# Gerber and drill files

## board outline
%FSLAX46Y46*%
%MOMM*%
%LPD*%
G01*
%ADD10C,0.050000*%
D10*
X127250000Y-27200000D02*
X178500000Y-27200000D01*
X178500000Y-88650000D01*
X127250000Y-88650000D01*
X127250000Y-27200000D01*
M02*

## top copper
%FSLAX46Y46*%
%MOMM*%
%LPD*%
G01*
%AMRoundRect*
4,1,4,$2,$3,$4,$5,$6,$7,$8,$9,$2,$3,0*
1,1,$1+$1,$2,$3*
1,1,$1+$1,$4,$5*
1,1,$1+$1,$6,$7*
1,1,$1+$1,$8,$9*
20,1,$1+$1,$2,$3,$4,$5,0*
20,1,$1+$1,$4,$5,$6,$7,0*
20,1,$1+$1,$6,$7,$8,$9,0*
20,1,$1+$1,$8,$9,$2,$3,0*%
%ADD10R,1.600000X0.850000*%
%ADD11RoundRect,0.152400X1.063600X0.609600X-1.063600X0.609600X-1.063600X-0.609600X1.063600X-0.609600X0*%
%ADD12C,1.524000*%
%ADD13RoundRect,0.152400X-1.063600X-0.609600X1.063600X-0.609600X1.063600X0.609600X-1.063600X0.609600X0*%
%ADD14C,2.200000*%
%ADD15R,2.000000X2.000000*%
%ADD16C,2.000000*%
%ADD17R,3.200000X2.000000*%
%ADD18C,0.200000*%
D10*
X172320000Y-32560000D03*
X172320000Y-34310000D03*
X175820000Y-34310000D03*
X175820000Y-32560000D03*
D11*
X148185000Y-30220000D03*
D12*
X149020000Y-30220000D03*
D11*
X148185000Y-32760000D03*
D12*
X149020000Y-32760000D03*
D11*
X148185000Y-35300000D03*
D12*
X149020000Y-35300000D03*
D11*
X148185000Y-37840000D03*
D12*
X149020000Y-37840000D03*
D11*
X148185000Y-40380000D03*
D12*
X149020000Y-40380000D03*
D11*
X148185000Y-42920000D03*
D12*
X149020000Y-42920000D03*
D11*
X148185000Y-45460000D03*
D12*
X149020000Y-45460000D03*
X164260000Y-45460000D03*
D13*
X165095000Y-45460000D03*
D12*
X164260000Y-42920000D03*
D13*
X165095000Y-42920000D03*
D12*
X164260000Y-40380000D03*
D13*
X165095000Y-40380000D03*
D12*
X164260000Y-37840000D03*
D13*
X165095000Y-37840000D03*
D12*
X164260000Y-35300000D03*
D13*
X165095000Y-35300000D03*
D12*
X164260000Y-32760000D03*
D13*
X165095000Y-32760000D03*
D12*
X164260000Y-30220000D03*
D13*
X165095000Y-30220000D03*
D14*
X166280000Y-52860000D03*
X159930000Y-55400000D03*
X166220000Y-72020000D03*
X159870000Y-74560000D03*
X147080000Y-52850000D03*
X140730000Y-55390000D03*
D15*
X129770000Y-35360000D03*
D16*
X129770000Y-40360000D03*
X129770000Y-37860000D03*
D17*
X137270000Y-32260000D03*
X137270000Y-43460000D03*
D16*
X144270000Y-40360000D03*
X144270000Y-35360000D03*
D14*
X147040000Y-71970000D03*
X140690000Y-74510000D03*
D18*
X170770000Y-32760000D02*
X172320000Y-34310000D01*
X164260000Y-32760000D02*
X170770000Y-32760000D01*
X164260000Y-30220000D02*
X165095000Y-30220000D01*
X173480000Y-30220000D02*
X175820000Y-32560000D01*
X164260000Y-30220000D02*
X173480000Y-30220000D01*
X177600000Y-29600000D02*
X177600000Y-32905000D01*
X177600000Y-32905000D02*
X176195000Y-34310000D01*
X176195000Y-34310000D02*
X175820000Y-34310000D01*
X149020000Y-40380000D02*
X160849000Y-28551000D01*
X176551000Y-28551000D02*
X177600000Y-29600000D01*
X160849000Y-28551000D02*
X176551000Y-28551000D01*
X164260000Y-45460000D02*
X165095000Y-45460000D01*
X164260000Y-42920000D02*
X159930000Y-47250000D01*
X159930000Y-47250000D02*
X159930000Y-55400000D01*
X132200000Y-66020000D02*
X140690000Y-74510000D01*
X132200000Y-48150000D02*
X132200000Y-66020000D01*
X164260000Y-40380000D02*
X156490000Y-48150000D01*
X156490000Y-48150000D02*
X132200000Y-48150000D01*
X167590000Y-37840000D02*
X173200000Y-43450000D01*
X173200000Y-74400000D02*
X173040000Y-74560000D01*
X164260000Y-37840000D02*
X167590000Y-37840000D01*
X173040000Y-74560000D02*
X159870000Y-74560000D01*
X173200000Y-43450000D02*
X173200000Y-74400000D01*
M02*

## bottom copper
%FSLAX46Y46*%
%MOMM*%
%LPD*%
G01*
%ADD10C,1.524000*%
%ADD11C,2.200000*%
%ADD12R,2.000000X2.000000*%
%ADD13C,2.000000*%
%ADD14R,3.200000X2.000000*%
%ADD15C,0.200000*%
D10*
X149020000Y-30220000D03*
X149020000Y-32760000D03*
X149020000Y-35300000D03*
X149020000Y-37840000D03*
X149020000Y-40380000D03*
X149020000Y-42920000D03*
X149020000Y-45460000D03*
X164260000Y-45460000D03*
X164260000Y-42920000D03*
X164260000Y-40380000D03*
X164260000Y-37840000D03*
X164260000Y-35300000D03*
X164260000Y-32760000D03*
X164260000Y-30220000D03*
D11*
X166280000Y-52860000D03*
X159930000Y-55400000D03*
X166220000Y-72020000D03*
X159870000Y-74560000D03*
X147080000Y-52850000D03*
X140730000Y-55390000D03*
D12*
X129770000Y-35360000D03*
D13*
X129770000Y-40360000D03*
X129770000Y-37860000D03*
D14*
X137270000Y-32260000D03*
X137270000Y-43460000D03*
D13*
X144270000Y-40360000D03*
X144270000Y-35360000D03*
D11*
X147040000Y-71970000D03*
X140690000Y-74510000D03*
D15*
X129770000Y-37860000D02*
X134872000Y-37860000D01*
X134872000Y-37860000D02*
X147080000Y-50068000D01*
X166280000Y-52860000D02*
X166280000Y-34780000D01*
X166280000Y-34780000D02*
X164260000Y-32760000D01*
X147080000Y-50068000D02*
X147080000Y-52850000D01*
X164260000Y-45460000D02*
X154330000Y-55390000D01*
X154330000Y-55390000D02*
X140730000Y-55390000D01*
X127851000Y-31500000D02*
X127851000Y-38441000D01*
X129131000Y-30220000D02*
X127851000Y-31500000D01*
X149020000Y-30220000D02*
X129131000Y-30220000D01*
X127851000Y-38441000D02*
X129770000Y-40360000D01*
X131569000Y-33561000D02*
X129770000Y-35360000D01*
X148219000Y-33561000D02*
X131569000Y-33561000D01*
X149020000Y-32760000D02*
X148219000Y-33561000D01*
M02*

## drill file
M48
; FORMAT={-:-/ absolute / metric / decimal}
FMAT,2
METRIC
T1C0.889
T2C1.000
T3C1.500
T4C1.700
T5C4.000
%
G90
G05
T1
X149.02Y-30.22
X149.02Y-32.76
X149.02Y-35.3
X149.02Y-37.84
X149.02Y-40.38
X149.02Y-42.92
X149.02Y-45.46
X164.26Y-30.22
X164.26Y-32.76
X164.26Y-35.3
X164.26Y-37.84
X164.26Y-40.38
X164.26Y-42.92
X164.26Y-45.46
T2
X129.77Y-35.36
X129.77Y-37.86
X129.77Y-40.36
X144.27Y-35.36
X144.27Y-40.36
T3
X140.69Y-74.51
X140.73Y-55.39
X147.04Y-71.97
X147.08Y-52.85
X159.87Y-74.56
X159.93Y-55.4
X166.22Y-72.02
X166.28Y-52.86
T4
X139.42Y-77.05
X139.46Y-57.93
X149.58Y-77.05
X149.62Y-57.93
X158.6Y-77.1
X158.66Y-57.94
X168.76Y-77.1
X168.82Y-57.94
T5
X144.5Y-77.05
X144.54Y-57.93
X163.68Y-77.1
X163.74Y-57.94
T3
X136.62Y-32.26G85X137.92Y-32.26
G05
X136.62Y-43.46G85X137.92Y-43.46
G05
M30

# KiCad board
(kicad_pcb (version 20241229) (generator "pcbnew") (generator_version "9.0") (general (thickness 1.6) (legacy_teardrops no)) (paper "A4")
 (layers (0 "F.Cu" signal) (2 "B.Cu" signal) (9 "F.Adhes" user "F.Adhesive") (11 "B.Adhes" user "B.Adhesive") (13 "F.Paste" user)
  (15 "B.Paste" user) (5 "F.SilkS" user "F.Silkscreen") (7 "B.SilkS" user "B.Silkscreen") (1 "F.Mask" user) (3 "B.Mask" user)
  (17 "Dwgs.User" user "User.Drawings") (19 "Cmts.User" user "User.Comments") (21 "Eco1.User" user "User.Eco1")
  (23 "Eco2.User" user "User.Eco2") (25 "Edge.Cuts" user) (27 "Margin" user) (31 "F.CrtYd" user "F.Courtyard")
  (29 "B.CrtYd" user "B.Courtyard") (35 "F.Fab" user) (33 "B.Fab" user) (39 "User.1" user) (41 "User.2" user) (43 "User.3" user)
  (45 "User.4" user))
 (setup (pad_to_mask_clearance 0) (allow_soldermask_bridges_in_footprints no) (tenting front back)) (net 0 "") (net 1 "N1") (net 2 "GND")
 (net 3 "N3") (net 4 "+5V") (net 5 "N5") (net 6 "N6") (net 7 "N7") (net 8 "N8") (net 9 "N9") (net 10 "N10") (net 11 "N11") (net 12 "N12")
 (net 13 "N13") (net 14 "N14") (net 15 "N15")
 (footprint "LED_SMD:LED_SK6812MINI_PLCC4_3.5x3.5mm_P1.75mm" (layer "F.Cu") (at 174.07 33.435)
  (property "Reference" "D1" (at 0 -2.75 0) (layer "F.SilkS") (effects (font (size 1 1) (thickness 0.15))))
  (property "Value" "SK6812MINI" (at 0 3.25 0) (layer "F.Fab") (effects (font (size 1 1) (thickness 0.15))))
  (pad "1" smd rect (at -1.75 -0.875) (size 1.6 0.85) (layers "F.Cu" "F.Mask" "F.Paste") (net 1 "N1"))
  (pad "2" smd rect (at -1.75 0.875) (size 1.6 0.85) (layers "F.Cu" "F.Mask" "F.Paste") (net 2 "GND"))
  (pad "3" smd rect (at 1.75 0.875) (size 1.6 0.85) (layers "F.Cu" "F.Mask" "F.Paste") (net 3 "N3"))
  (pad "4" smd rect (at 1.75 -0.875) (size 1.6 0.85) (layers "F.Cu" "F.Mask" "F.Paste") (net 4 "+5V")))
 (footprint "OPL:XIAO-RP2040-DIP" (layer "F.Cu") (at 156.64 37.84)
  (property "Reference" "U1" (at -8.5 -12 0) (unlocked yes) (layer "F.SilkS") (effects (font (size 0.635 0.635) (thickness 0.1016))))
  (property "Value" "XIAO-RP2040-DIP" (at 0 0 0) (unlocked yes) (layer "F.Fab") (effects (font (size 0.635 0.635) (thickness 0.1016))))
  (pad "1" smd roundrect (at -8.455 -7.62 180) (size 2.432 1.524) (layers "F.Cu" "F.Mask") (roundrect_rratio 0.1) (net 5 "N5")
   (thermal_bridge_angle 45))
  (pad "1" thru_hole circle (at -7.62 -7.62 180) (size 1.524 1.524) (drill 0.889) (layers "*.Cu" "*.Mask") (remove_unused_layers no)
   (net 5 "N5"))
  (pad "2" smd roundrect (at -8.455 -5.08 180) (size 2.432 1.524) (layers "F.Cu" "F.Mask") (roundrect_rratio 0.1) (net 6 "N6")
   (thermal_bridge_angle 45))
  (pad "2" thru_hole circle (at -7.62 -5.08 180) (size 1.524 1.524) (drill 0.889) (layers "*.Cu" "*.Mask") (remove_unused_layers no)
   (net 6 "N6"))
  (pad "3" smd roundrect (at -8.455 -2.54 180) (size 2.432 1.524) (layers "F.Cu" "F.Mask") (roundrect_rratio 0.1) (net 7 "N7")
   (thermal_bridge_angle 45))
  (pad "3" thru_hole circle (at -7.62 -2.54 180) (size 1.524 1.524) (drill 0.889) (layers "*.Cu" "*.Mask") (remove_unused_layers no)
   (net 7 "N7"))
  (pad "4" smd roundrect (at -8.455 0 180) (size 2.432 1.524) (layers "F.Cu" "F.Mask") (roundrect_rratio 0.1) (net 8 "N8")
   (thermal_bridge_angle 45))
  (pad "4" thru_hole circle (at -7.62 0 180) (size 1.524 1.524) (drill 0.889) (layers "*.Cu" "*.Mask") (remove_unused_layers no)
   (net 8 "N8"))
  (pad "5" smd roundrect (at -8.455 2.54 180) (size 2.432 1.524) (layers "F.Cu" "F.Mask") (roundrect_rratio 0.1) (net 3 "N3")
   (thermal_bridge_angle 45))
  (pad "5" thru_hole circle (at -7.62 2.54 180) (size 1.524 1.524) (drill 0.889) (layers "*.Cu" "*.Mask") (remove_unused_layers no)
   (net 3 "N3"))
  (pad "6" smd roundrect (at -8.455 5.08 180) (size 2.432 1.524) (layers "F.Cu" "F.Mask") (roundrect_rratio 0.1) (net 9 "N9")
   (thermal_bridge_angle 45))
  (pad "6" thru_hole circle (at -7.62 5.08 180) (size 1.524 1.524) (drill 0.889) (layers "*.Cu" "*.Mask") (remove_unused_layers no)
   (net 9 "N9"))
  (pad "7" smd roundrect (at -8.455 7.62 180) (size 2.432 1.524) (layers "F.Cu" "F.Mask") (roundrect_rratio 0.1) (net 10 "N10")
   (thermal_bridge_angle 45))
  (pad "7" thru_hole circle (at -7.62 7.62 180) (size 1.524 1.524) (drill 0.889) (layers "*.Cu" "*.Mask") (remove_unused_layers no)
   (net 10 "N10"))
  (pad "8" thru_hole circle (at 7.62 7.62) (size 1.524 1.524) (drill 0.889) (layers "*.Cu" "*.Mask") (remove_unused_layers no)
   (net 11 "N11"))
  (pad "8" smd roundrect (at 8.455 7.62) (size 2.432 1.524) (layers "F.Cu" "F.Mask") (roundrect_rratio 0.1) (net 11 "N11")
   (thermal_bridge_angle 45))
  (pad "9" thru_hole circle (at 7.62 5.08) (size 1.524 1.524) (drill 0.889) (layers "*.Cu" "*.Mask") (remove_unused_layers no)
   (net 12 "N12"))
  (pad "9" smd roundrect (at 8.455 5.08) (size 2.432 1.524) (layers "F.Cu" "F.Mask") (roundrect_rratio 0.1) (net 12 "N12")
   (thermal_bridge_angle 45))
  (pad "10" thru_hole circle (at 7.62 2.54) (size 1.524 1.524) (drill 0.889) (layers "*.Cu" "*.Mask") (remove_unused_layers no)
   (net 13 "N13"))
  (pad "10" smd roundrect (at 8.455 2.54) (size 2.432 1.524) (layers "F.Cu" "F.Mask") (roundrect_rratio 0.1) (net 13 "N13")
   (thermal_bridge_angle 45))
  (pad "11" thru_hole circle (at 7.62 0) (size 1.524 1.524) (drill 0.889) (layers "*.Cu" "*.Mask") (remove_unused_layers no) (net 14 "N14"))
  (pad "11" smd roundrect (at 8.455 0) (size 2.432 1.524) (layers "F.Cu" "F.Mask") (roundrect_rratio 0.1) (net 14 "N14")
   (thermal_bridge_angle 45))
  (pad "12" thru_hole circle (at 7.62 -2.54) (size 1.524 1.524) (drill 0.889) (layers "*.Cu" "*.Mask") (remove_unused_layers no)
   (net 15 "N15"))
  (pad "12" smd roundrect (at 8.455 -2.54) (size 2.432 1.524) (layers "F.Cu" "F.Mask") (roundrect_rratio 0.1) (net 15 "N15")
   (thermal_bridge_angle 45))
  (pad "13" thru_hole circle (at 7.62 -5.08) (size 1.524 1.524) (drill 0.889) (layers "*.Cu" "*.Mask") (remove_unused_layers no)
   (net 2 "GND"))
  (pad "13" smd roundrect (at 8.455 -5.08) (size 2.432 1.524) (layers "F.Cu" "F.Mask") (roundrect_rratio 0.1) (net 2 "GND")
   (thermal_bridge_angle 45))
  (pad "14" thru_hole circle (at 7.62 -7.62) (size 1.524 1.524) (drill 0.889) (layers "*.Cu" "*.Mask") (remove_unused_layers no)
   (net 4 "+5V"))
  (pad "14" smd roundrect (at 8.455 -7.62) (size 2.432 1.524) (layers "F.Cu" "F.Mask") (roundrect_rratio 0.1) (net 4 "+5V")
   (thermal_bridge_angle 45)))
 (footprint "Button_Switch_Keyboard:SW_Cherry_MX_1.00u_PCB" (layer "F.Cu") (at 166.28 52.86)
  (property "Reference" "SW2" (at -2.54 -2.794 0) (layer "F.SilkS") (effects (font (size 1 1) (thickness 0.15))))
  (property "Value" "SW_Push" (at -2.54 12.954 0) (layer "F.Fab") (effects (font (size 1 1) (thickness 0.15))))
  (pad "" np_thru_hole circle (at -7.62 5.08) (size 1.7 1.7) (drill 1.7) (layers "*.Cu" "*.Mask"))
  (pad "" np_thru_hole circle (at -2.54 5.08) (size 4 4) (drill 4) (layers "*.Cu" "*.Mask"))
  (pad "" np_thru_hole circle (at 2.54 5.08) (size 1.7 1.7) (drill 1.7) (layers "*.Cu" "*.Mask"))
  (pad "1" thru_hole circle (at 0 0) (size 2.2 2.2) (drill 1.5) (layers "*.Cu" "*.Mask") (remove_unused_layers no) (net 2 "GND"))
  (pad "2" thru_hole circle (at -6.35 2.54) (size 2.2 2.2) (drill 1.5) (layers "*.Cu" "*.Mask") (remove_unused_layers no) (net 12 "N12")))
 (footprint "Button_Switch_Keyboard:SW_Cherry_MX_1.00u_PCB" (layer "F.Cu") (at 166.22 72.02)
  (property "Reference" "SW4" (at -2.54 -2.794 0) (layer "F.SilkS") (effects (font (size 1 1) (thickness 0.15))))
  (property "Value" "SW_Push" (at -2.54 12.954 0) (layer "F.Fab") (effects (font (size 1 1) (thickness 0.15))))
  (pad "" np_thru_hole circle (at -7.62 5.08) (size 1.7 1.7) (drill 1.7) (layers "*.Cu" "*.Mask"))
  (pad "" np_thru_hole circle (at -2.54 5.08) (size 4 4) (drill 4) (layers "*.Cu" "*.Mask"))
  (pad "" np_thru_hole circle (at 2.54 5.08) (size 1.7 1.7) (drill 1.7) (layers "*.Cu" "*.Mask"))
  (pad "1" thru_hole circle (at 0 0) (size 2.2 2.2) (drill 1.5) (layers "*.Cu" "*.Mask") (remove_unused_layers no) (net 2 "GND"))
  (pad "2" thru_hole circle (at -6.35 2.54) (size 2.2 2.2) (drill 1.5) (layers "*.Cu" "*.Mask") (remove_unused_layers no) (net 14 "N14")))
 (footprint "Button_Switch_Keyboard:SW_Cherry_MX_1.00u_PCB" (layer "F.Cu") (at 147.08 52.85)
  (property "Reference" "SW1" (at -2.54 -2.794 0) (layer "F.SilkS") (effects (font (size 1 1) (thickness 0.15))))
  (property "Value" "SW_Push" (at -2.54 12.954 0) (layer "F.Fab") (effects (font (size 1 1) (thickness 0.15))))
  (pad "" np_thru_hole circle (at -7.62 5.08) (size 1.7 1.7) (drill 1.7) (layers "*.Cu" "*.Mask"))
  (pad "" np_thru_hole circle (at -2.54 5.08) (size 4 4) (drill 4) (layers "*.Cu" "*.Mask"))
  (pad "" np_thru_hole circle (at 2.54 5.08) (size 1.7 1.7) (drill 1.7) (layers "*.Cu" "*.Mask"))
  (pad "1" thru_hole circle (at 0 0) (size 2.2 2.2) (drill 1.5) (layers "*.Cu" "*.Mask") (remove_unused_layers no) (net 2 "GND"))
  (pad "2" thru_hole circle (at -6.35 2.54) (size 2.2 2.2) (drill 1.5) (layers "*.Cu" "*.Mask") (remove_unused_layers no) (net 11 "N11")))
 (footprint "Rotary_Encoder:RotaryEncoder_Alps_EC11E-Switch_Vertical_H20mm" (layer "F.Cu") (at 129.77 35.36)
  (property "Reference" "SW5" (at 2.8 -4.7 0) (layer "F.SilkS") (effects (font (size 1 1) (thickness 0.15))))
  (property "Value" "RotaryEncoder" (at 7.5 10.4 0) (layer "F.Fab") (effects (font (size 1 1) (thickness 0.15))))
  (pad "A" thru_hole rect (at 0 0) (size 2 2) (drill 1) (layers "*.Cu" "*.Mask") (remove_unused_layers no) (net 6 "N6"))
  (pad "B" thru_hole circle (at 0 5) (size 2 2) (drill 1) (layers "*.Cu" "*.Mask") (remove_unused_layers no) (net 5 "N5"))
  (pad "C" thru_hole circle (at 0 2.5) (size 2 2) (drill 1) (layers "*.Cu" "*.Mask") (remove_unused_layers no) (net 2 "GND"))
  (pad "MP" thru_hole rect (at 7.5 -3.1) (size 3.2 2) (drill oval 2.8 1.5) (layers "*.Cu" "*.Mask") (remove_unused_layers no))
  (pad "MP" thru_hole rect (at 7.5 8.1) (size 3.2 2) (drill oval 2.8 1.5) (layers "*.Cu" "*.Mask") (remove_unused_layers no))
  (pad "S1" thru_hole circle (at 14.5 5) (size 2 2) (drill 1) (layers "*.Cu" "*.Mask") (remove_unused_layers no))
  (pad "S2" thru_hole circle (at 14.5 0) (size 2 2) (drill 1) (layers "*.Cu" "*.Mask") (remove_unused_layers no)))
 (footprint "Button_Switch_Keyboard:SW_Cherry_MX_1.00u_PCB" (layer "F.Cu") (at 147.04 71.97)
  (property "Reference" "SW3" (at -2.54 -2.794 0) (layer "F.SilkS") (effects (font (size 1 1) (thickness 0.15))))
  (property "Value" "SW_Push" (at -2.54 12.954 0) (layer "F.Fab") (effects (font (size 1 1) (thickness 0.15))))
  (pad "" np_thru_hole circle (at -7.62 5.08) (size 1.7 1.7) (drill 1.7) (layers "*.Cu" "*.Mask"))
  (pad "" np_thru_hole circle (at -2.54 5.08) (size 4 4) (drill 4) (layers "*.Cu" "*.Mask"))
  (pad "" np_thru_hole circle (at 2.54 5.08) (size 1.7 1.7) (drill 1.7) (layers "*.Cu" "*.Mask"))
  (pad "1" thru_hole circle (at 0 0) (size 2.2 2.2) (drill 1.5) (layers "*.Cu" "*.Mask") (remove_unused_layers no) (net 2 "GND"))
  (pad "2" thru_hole circle (at -6.35 2.54) (size 2.2 2.2) (drill 1.5) (layers "*.Cu" "*.Mask") (remove_unused_layers no) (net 13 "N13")))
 (gr_rect (start 127.25 27.2) (end 178.5 88.65) (stroke (width 0.05) (type default)) (fill no) (layer "Edge.Cuts"))
 (segment (start 170.77 32.76) (end 172.32 34.31) (width 0.2) (layer "F.Cu") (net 2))
 (segment (start 164.26 32.76) (end 170.77 32.76) (width 0.2) (layer "F.Cu") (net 2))
 (segment (start 129.77 37.86) (end 134.872 37.86) (width 0.2) (layer "B.Cu") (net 2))
 (segment (start 134.872 37.86) (end 147.08 50.068) (width 0.2) (layer "B.Cu") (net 2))
 (segment (start 166.28 52.86) (end 166.28 34.78) (width 0.2) (layer "B.Cu") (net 2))
 (segment (start 166.28 34.78) (end 164.26 32.76) (width 0.2) (layer "B.Cu") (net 2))
 (segment (start 147.08 50.068) (end 147.08 52.85) (width 0.2) (layer "B.Cu") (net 2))
 (segment (start 164.26 30.22) (end 165.095 30.22) (width 0.2) (layer "F.Cu") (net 4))
 (segment (start 173.48 30.22) (end 175.82 32.56) (width 0.2) (layer "F.Cu") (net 4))
 (segment (start 164.26 30.22) (end 173.48 30.22) (width 0.2) (layer "F.Cu") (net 4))
 (segment (start 177.6 29.6) (end 177.6 32.905) (width 0.2) (layer "F.Cu") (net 3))
 (segment (start 177.6 32.905) (end 176.195 34.31) (width 0.2) (layer "F.Cu") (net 3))
 (segment (start 176.195 34.31) (end 175.82 34.31) (width 0.2) (layer "F.Cu") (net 3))
 (segment (start 149.02 40.38) (end 160.849 28.551) (width 0.2) (layer "F.Cu") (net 3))
 (segment (start 176.551 28.551) (end 177.6 29.6) (width 0.2) (layer "F.Cu") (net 3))
 (segment (start 160.849 28.551) (end 176.551 28.551) (width 0.2) (layer "F.Cu") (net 3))
 (segment (start 164.26 45.46) (end 165.095 45.46) (width 0.2) (layer "F.Cu") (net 11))
 (segment (start 164.26 45.46) (end 154.33 55.39) (width 0.2) (layer "B.Cu") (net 11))
 (segment (start 154.33 55.39) (end 140.73 55.39) (width 0.2) (layer "B.Cu") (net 11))
 (segment (start 164.26 42.92) (end 159.93 47.25) (width 0.2) (layer "F.Cu") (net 12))
 (segment (start 159.93 47.25) (end 159.93 55.4) (width 0.2) (layer "F.Cu") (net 12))
 (segment (start 132.2 66.02) (end 140.69 74.51) (width 0.2) (layer "F.Cu") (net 13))
 (segment (start 132.2 48.15) (end 132.2 66.02) (width 0.2) (layer "F.Cu") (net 13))
 (segment (start 164.26 40.38) (end 156.49 48.15) (width 0.2) (layer "F.Cu") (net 13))
 (segment (start 156.49 48.15) (end 132.2 48.15) (width 0.2) (layer "F.Cu") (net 13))
 (segment (start 167.59 37.84) (end 173.2 43.45) (width 0.2) (layer "F.Cu") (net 14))
 (segment (start 173.2 74.4) (end 173.04 74.56) (width 0.2) (layer "F.Cu") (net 14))
 (segment (start 164.26 37.84) (end 167.59 37.84) (width 0.2) (layer "F.Cu") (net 14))
 (segment (start 173.04 74.56) (end 159.87 74.56) (width 0.2) (layer "F.Cu") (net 14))
 (segment (start 173.2 43.45) (end 173.2 74.4) (width 0.2) (layer "F.Cu") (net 14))
 (segment (start 127.851 31.5) (end 127.851 38.441) (width 0.2) (layer "B.Cu") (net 5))
 (segment (start 129.131 30.22) (end 127.851 31.5) (width 0.2) (layer "B.Cu") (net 5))
 (segment (start 149.02 30.22) (end 129.131 30.22) (width 0.2) (layer "B.Cu") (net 5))
 (segment (start 127.851 38.441) (end 129.77 40.36) (width 0.2) (layer "B.Cu") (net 5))
 (segment (start 131.569 33.561) (end 129.77 35.36) (width 0.2) (layer "B.Cu") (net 6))
 (segment (start 148.219 33.561) (end 131.569 33.561) (width 0.2) (layer "B.Cu") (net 6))
 (segment (start 149.02 32.76) (end 148.219 33.561) (width 0.2) (layer "B.Cu") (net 6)))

